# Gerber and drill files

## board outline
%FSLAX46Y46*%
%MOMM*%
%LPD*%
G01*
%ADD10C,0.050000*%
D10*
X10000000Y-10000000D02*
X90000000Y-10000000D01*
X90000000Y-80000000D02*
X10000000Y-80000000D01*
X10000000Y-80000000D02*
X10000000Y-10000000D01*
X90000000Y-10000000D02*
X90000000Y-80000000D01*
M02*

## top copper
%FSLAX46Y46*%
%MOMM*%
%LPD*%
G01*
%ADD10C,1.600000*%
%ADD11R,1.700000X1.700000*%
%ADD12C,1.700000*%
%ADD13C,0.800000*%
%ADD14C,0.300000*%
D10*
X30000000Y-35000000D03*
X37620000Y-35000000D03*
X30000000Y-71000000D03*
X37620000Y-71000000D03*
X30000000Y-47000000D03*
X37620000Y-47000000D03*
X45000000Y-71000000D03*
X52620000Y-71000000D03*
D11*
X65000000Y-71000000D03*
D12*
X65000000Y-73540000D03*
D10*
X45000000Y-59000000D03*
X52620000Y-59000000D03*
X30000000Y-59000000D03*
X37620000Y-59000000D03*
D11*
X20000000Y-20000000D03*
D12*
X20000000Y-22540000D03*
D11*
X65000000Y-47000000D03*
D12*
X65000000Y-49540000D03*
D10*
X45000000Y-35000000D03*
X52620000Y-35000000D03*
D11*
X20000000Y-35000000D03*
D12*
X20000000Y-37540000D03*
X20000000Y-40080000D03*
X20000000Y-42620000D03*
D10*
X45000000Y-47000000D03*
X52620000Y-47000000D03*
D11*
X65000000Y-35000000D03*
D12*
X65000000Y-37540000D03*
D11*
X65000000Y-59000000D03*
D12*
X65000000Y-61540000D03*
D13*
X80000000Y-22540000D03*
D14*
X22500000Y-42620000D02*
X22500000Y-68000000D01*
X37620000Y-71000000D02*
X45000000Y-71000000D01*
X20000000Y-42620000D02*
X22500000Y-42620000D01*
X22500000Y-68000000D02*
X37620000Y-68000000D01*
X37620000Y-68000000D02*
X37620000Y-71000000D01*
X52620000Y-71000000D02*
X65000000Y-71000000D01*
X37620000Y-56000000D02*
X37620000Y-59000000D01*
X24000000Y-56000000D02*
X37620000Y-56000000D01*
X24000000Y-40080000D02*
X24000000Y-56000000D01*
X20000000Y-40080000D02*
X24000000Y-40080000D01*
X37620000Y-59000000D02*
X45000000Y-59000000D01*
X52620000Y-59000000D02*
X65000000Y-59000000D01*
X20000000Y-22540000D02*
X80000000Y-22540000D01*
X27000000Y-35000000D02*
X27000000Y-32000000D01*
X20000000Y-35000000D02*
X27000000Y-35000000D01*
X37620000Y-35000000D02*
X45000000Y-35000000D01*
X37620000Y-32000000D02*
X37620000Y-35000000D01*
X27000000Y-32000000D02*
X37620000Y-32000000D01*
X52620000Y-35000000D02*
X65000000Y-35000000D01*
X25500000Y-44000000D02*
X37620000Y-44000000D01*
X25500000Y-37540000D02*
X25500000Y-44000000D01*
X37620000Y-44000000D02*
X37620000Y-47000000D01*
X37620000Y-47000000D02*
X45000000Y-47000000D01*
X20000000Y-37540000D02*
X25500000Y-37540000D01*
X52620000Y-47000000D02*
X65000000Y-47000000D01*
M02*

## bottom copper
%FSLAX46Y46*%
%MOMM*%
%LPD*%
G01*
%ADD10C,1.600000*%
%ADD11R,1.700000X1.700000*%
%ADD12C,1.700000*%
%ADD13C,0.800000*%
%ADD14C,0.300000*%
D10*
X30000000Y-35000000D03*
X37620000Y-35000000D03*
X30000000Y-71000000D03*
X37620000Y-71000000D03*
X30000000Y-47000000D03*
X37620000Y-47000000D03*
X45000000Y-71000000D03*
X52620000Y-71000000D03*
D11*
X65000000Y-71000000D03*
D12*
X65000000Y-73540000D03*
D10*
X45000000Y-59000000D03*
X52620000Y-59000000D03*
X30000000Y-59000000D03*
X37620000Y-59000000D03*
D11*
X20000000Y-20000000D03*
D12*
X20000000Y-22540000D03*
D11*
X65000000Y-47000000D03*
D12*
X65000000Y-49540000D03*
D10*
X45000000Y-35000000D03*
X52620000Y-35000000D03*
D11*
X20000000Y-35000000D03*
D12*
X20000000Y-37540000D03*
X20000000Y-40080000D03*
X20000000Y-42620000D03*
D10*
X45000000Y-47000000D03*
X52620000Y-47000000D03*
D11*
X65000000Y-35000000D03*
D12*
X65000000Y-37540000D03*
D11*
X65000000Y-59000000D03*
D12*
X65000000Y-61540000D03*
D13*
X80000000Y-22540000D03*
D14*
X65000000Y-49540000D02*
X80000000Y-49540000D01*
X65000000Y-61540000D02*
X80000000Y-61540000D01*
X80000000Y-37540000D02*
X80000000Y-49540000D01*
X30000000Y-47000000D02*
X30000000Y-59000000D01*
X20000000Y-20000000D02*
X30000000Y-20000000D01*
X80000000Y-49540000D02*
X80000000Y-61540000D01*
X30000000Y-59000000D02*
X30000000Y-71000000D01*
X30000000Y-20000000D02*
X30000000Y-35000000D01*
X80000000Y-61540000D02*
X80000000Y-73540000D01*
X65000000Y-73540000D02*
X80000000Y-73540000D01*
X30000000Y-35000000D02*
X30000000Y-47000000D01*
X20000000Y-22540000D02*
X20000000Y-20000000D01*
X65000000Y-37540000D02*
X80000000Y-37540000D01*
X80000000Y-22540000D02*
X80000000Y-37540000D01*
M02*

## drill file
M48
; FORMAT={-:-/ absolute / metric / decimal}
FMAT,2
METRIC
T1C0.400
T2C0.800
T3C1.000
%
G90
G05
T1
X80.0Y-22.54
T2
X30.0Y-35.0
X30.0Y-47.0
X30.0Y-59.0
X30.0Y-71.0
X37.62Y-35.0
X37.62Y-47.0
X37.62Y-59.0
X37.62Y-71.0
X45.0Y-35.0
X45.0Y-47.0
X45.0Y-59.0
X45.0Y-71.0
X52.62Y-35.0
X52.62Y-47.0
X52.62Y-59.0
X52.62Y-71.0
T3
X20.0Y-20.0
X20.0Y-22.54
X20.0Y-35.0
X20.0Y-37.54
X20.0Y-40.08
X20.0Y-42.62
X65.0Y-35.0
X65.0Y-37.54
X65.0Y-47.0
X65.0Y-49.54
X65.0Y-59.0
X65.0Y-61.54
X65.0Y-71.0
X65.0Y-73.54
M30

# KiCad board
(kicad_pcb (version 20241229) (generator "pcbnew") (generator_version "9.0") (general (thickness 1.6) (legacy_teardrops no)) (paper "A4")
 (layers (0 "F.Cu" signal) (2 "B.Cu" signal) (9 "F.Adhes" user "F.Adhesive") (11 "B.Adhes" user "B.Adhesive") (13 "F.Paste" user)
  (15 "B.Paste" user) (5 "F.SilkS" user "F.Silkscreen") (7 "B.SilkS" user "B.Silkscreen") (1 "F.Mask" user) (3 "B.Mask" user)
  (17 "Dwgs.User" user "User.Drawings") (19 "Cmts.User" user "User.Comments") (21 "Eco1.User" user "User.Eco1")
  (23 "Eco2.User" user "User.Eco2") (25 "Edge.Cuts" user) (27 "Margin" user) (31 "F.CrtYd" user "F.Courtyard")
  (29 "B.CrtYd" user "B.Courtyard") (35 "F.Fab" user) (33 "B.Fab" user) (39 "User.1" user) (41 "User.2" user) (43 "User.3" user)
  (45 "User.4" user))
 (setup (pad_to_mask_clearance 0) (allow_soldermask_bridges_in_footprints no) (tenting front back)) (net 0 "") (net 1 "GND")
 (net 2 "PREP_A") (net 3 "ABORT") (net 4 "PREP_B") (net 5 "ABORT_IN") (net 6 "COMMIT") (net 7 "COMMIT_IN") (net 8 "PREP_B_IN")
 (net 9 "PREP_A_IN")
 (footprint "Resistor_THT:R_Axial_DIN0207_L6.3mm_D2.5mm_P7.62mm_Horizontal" (layer "F.Cu") (at 30 35)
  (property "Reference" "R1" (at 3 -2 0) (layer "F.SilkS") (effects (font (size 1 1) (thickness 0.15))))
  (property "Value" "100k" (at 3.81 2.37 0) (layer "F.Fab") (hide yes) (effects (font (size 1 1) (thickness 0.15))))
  (pad "1" thru_hole circle (at 0 0) (size 1.6 1.6) (drill 0.8) (layers "*.Cu" "*.Mask") (remove_unused_layers no) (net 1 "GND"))
  (pad "2" thru_hole circle (at 7.62 0) (size 1.6 1.6) (drill 0.8) (layers "*.Cu" "*.Mask") (remove_unused_layers no) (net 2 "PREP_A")))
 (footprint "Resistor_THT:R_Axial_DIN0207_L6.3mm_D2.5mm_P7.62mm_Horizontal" (layer "F.Cu") (at 30 71)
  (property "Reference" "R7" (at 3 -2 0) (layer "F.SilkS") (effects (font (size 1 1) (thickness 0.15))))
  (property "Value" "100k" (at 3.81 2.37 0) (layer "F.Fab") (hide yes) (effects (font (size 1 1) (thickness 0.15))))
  (pad "1" thru_hole circle (at 0 0) (size 1.6 1.6) (drill 0.8) (layers "*.Cu" "*.Mask") (remove_unused_layers no) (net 1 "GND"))
  (pad "2" thru_hole circle (at 7.62 0) (size 1.6 1.6) (drill 0.8) (layers "*.Cu" "*.Mask") (remove_unused_layers no) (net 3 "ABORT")))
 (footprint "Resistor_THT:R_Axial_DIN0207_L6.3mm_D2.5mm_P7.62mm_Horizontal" (layer "F.Cu") (at 30 47)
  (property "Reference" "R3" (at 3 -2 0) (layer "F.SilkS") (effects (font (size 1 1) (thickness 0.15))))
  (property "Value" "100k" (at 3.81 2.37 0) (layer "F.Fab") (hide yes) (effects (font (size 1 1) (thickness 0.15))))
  (pad "1" thru_hole circle (at 0 0) (size 1.6 1.6) (drill 0.8) (layers "*.Cu" "*.Mask") (remove_unused_layers no) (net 1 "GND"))
  (pad "2" thru_hole circle (at 7.62 0) (size 1.6 1.6) (drill 0.8) (layers "*.Cu" "*.Mask") (remove_unused_layers no) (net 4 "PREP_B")))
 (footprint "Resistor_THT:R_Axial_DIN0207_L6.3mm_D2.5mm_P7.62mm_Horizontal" (layer "F.Cu") (at 45 71)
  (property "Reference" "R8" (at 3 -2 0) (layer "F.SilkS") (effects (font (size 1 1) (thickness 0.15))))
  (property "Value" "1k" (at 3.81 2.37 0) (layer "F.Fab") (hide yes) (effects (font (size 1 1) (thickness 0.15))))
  (pad "1" thru_hole circle (at 0 0) (size 1.6 1.6) (drill 0.8) (layers "*.Cu" "*.Mask") (remove_unused_layers no) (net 3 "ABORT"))
  (pad "2" thru_hole circle (at 7.62 0) (size 1.6 1.6) (drill 0.8) (layers "*.Cu" "*.Mask") (remove_unused_layers no) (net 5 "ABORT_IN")))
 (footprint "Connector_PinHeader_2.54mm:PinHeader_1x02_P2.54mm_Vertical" (layer "F.Cu") (at 65 71)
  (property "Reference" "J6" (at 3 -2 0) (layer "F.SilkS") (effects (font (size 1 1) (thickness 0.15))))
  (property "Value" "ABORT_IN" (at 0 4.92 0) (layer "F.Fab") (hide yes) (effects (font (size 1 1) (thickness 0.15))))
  (pad "1" thru_hole rect (at 0 0) (size 1.7 1.7) (drill 1) (layers "*.Cu" "*.Mask") (remove_unused_layers no) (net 5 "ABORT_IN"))
  (pad "2" thru_hole circle (at 0 2.54) (size 1.7 1.7) (drill 1) (layers "*.Cu" "*.Mask") (remove_unused_layers no) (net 1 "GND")))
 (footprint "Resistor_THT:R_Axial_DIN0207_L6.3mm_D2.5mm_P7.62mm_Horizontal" (layer "F.Cu") (at 45 59)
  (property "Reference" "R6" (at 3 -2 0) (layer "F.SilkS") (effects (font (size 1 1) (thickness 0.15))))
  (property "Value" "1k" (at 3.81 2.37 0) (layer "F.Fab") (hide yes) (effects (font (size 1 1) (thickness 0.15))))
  (pad "1" thru_hole circle (at 0 0) (size 1.6 1.6) (drill 0.8) (layers "*.Cu" "*.Mask") (remove_unused_layers no) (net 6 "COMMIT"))
  (pad "2" thru_hole circle (at 7.62 0) (size 1.6 1.6) (drill 0.8) (layers "*.Cu" "*.Mask") (remove_unused_layers no) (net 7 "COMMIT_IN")))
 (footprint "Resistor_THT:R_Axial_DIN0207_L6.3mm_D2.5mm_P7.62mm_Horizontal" (layer "F.Cu") (at 30 59)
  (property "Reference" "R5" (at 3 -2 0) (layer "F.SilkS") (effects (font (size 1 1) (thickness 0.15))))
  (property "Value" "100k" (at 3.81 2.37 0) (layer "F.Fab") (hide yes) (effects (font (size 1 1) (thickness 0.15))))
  (pad "1" thru_hole circle (at 0 0) (size 1.6 1.6) (drill 0.8) (layers "*.Cu" "*.Mask") (remove_unused_layers no) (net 1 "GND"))
  (pad "2" thru_hole circle (at 7.62 0) (size 1.6 1.6) (drill 0.8) (layers "*.Cu" "*.Mask") (remove_unused_layers no) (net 6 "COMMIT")))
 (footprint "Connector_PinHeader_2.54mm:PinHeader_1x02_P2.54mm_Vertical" (layer "F.Cu") (at 20 20)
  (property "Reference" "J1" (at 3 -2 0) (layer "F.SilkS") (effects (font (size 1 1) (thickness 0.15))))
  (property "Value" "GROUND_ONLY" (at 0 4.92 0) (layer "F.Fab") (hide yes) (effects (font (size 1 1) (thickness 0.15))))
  (pad "1" thru_hole rect (at 0 0) (size 1.7 1.7) (drill 1) (layers "*.Cu" "*.Mask") (remove_unused_layers no) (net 1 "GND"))
  (pad "2" thru_hole circle (at 0 2.54) (size 1.7 1.7) (drill 1) (layers "*.Cu" "*.Mask") (remove_unused_layers no) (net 1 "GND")))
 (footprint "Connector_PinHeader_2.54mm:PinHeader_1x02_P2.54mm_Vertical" (layer "F.Cu") (at 65 47)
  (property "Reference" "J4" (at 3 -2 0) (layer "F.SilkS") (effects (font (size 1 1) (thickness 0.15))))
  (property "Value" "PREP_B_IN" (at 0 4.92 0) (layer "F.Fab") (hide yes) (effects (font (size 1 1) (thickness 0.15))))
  (pad "1" thru_hole rect (at 0 0) (size 1.7 1.7) (drill 1) (layers "*.Cu" "*.Mask") (remove_unused_layers no) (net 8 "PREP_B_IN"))
  (pad "2" thru_hole circle (at 0 2.54) (size 1.7 1.7) (drill 1) (layers "*.Cu" "*.Mask") (remove_unused_layers no) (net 1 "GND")))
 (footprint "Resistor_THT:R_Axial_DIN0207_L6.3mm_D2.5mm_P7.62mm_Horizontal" (layer "F.Cu") (at 45 35)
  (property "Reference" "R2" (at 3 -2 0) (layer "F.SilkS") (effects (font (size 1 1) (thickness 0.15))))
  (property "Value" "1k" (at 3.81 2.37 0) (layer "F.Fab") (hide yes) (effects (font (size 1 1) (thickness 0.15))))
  (pad "1" thru_hole circle (at 0 0) (size 1.6 1.6) (drill 0.8) (layers "*.Cu" "*.Mask") (remove_unused_layers no) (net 2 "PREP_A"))
  (pad "2" thru_hole circle (at 7.62 0) (size 1.6 1.6) (drill 0.8) (layers "*.Cu" "*.Mask") (remove_unused_layers no) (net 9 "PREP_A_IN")))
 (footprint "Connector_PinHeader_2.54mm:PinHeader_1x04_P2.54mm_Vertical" (layer "F.Cu") (at 20 35)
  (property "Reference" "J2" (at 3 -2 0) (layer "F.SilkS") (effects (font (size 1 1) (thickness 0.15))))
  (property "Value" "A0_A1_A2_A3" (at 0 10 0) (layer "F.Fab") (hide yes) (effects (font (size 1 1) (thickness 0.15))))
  (pad "1" thru_hole rect (at 0 0) (size 1.7 1.7) (drill 1) (layers "*.Cu" "*.Mask") (remove_unused_layers no) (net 2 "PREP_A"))
  (pad "2" thru_hole circle (at 0 2.54) (size 1.7 1.7) (drill 1) (layers "*.Cu" "*.Mask") (remove_unused_layers no) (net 4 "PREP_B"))
  (pad "3" thru_hole circle (at 0 5.08) (size 1.7 1.7) (drill 1) (layers "*.Cu" "*.Mask") (remove_unused_layers no) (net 6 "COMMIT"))
  (pad "4" thru_hole circle (at 0 7.62) (size 1.7 1.7) (drill 1) (layers "*.Cu" "*.Mask") (remove_unused_layers no) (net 3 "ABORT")))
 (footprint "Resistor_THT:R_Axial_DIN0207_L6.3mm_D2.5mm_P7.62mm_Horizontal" (layer "F.Cu") (at 45 47)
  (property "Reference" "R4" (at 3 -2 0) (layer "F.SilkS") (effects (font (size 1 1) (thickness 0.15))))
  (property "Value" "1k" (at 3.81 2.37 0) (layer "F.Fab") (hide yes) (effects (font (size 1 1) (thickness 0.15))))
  (pad "1" thru_hole circle (at 0 0) (size 1.6 1.6) (drill 0.8) (layers "*.Cu" "*.Mask") (remove_unused_layers no) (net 4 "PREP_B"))
  (pad "2" thru_hole circle (at 7.62 0) (size 1.6 1.6) (drill 0.8) (layers "*.Cu" "*.Mask") (remove_unused_layers no) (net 8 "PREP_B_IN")))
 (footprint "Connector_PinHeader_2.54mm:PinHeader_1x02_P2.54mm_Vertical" (layer "F.Cu") (at 65 35)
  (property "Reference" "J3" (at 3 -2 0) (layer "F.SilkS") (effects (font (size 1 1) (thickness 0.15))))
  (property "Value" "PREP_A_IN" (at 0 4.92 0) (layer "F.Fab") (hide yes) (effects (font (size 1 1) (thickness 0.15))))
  (pad "1" thru_hole rect (at 0 0) (size 1.7 1.7) (drill 1) (layers "*.Cu" "*.Mask") (remove_unused_layers no) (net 9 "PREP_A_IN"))
  (pad "2" thru_hole circle (at 0 2.54) (size 1.7 1.7) (drill 1) (layers "*.Cu" "*.Mask") (remove_unused_layers no) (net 1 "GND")))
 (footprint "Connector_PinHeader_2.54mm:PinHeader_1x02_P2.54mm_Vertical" (layer "F.Cu") (at 65 59)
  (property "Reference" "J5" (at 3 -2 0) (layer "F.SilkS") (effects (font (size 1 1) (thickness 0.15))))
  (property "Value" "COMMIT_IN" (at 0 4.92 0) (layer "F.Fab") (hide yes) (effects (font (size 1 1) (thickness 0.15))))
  (pad "1" thru_hole rect (at 0 0) (size 1.7 1.7) (drill 1) (layers "*.Cu" "*.Mask") (remove_unused_layers no) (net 7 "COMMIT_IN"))
  (pad "2" thru_hole circle (at 0 2.54) (size 1.7 1.7) (drill 1) (layers "*.Cu" "*.Mask") (remove_unused_layers no) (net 1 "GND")))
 (gr_line (start 10 10) (end 90 10) (stroke (width 0.05) (type default)) (layer "Edge.Cuts"))
 (gr_line (start 90 80) (end 10 80) (stroke (width 0.05) (type default)) (layer "Edge.Cuts"))
 (gr_line (start 10 80) (end 10 10) (stroke (width 0.05) (type default)) (layer "Edge.Cuts"))
 (gr_line (start 90 10) (end 90 80) (stroke (width 0.05) (type default)) (layer "Edge.Cuts"))
 (segment (start 22.5 42.62) (end 22.5 68) (width 0.3) (layer "F.Cu") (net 3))
 (segment (start 37.62 71) (end 45 71) (width 0.3) (layer "F.Cu") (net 3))
 (segment (start 20 42.62) (end 22.5 42.62) (width 0.3) (layer "F.Cu") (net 3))
 (segment (start 22.5 68) (end 37.62 68) (width 0.3) (layer "F.Cu") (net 3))
 (segment (start 37.62 68) (end 37.62 71) (width 0.3) (layer "F.Cu") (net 3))
 (segment (start 52.62 71) (end 65 71) (width 0.3) (layer "F.Cu") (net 5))
 (segment (start 37.62 56) (end 37.62 59) (width 0.3) (layer "F.Cu") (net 6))
 (segment (start 24 56) (end 37.62 56) (width 0.3) (layer "F.Cu") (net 6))
 (segment (start 24 40.08) (end 24 56) (width 0.3) (layer "F.Cu") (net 6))
 (segment (start 20 40.08) (end 24 40.08) (width 0.3) (layer "F.Cu") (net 6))
 (segment (start 37.62 59) (end 45 59) (width 0.3) (layer "F.Cu") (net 6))
 (segment (start 52.62 59) (end 65 59) (width 0.3) (layer "F.Cu") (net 7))
 (segment (start 20 22.54) (end 80 22.54) (width 0.3) (layer "F.Cu") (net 1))
 (via (at 80 22.54) (size 0.8) (drill 0.4) (layers "F.Cu" "B.Cu") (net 1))
 (segment (start 65 49.54) (end 80 49.54) (width 0.3) (layer "B.Cu") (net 1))
 (segment (start 65 61.54) (end 80 61.54) (width 0.3) (layer "B.Cu") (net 1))
 (segment (start 80 37.54) (end 80 49.54) (width 0.3) (layer "B.Cu") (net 1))
 (segment (start 30 47) (end 30 59) (width 0.3) (layer "B.Cu") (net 1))
 (segment (start 20 20) (end 30 20) (width 0.3) (layer "B.Cu") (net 1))
 (segment (start 80 49.54) (end 80 61.54) (width 0.3) (layer "B.Cu") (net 1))
 (segment (start 30 59) (end 30 71) (width 0.3) (layer "B.Cu") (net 1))
 (segment (start 30 20) (end 30 35) (width 0.3) (layer "B.Cu") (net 1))
 (segment (start 80 61.54) (end 80 73.54) (width 0.3) (layer "B.Cu") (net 1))
 (segment (start 65 73.54) (end 80 73.54) (width 0.3) (layer "B.Cu") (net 1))
 (segment (start 30 35) (end 30 47) (width 0.3) (layer "B.Cu") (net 1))
 (segment (start 20 22.54) (end 20 20) (width 0.3) (layer "B.Cu") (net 1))
 (segment (start 65 37.54) (end 80 37.54) (width 0.3) (layer "B.Cu") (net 1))
 (segment (start 80 22.54) (end 80 37.54) (width 0.3) (layer "B.Cu") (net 1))
 (segment (start 27 35) (end 27 32) (width 0.3) (layer "F.Cu") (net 2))
 (segment (start 20 35) (end 27 35) (width 0.3) (layer "F.Cu") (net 2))
 (segment (start 37.62 35) (end 45 35) (width 0.3) (layer "F.Cu") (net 2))
 (segment (start 37.62 32) (end 37.62 35) (width 0.3) (layer "F.Cu") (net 2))
 (segment (start 27 32) (end 37.62 32) (width 0.3) (layer "F.Cu") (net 2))
 (segment (start 52.62 35) (end 65 35) (width 0.3) (layer "F.Cu") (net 9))
 (segment (start 25.5 44) (end 37.62 44) (width 0.3) (layer "F.Cu") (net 4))
 (segment (start 25.5 37.54) (end 25.5 44) (width 0.3) (layer "F.Cu") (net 4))
 (segment (start 37.62 44) (end 37.62 47) (width 0.3) (layer "F.Cu") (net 4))
 (segment (start 37.62 47) (end 45 47) (width 0.3) (layer "F.Cu") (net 4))
 (segment (start 20 37.54) (end 25.5 37.54) (width 0.3) (layer "F.Cu") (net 4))
 (segment (start 52.62 47) (end 65 47) (width 0.3) (layer "F.Cu") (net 8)))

